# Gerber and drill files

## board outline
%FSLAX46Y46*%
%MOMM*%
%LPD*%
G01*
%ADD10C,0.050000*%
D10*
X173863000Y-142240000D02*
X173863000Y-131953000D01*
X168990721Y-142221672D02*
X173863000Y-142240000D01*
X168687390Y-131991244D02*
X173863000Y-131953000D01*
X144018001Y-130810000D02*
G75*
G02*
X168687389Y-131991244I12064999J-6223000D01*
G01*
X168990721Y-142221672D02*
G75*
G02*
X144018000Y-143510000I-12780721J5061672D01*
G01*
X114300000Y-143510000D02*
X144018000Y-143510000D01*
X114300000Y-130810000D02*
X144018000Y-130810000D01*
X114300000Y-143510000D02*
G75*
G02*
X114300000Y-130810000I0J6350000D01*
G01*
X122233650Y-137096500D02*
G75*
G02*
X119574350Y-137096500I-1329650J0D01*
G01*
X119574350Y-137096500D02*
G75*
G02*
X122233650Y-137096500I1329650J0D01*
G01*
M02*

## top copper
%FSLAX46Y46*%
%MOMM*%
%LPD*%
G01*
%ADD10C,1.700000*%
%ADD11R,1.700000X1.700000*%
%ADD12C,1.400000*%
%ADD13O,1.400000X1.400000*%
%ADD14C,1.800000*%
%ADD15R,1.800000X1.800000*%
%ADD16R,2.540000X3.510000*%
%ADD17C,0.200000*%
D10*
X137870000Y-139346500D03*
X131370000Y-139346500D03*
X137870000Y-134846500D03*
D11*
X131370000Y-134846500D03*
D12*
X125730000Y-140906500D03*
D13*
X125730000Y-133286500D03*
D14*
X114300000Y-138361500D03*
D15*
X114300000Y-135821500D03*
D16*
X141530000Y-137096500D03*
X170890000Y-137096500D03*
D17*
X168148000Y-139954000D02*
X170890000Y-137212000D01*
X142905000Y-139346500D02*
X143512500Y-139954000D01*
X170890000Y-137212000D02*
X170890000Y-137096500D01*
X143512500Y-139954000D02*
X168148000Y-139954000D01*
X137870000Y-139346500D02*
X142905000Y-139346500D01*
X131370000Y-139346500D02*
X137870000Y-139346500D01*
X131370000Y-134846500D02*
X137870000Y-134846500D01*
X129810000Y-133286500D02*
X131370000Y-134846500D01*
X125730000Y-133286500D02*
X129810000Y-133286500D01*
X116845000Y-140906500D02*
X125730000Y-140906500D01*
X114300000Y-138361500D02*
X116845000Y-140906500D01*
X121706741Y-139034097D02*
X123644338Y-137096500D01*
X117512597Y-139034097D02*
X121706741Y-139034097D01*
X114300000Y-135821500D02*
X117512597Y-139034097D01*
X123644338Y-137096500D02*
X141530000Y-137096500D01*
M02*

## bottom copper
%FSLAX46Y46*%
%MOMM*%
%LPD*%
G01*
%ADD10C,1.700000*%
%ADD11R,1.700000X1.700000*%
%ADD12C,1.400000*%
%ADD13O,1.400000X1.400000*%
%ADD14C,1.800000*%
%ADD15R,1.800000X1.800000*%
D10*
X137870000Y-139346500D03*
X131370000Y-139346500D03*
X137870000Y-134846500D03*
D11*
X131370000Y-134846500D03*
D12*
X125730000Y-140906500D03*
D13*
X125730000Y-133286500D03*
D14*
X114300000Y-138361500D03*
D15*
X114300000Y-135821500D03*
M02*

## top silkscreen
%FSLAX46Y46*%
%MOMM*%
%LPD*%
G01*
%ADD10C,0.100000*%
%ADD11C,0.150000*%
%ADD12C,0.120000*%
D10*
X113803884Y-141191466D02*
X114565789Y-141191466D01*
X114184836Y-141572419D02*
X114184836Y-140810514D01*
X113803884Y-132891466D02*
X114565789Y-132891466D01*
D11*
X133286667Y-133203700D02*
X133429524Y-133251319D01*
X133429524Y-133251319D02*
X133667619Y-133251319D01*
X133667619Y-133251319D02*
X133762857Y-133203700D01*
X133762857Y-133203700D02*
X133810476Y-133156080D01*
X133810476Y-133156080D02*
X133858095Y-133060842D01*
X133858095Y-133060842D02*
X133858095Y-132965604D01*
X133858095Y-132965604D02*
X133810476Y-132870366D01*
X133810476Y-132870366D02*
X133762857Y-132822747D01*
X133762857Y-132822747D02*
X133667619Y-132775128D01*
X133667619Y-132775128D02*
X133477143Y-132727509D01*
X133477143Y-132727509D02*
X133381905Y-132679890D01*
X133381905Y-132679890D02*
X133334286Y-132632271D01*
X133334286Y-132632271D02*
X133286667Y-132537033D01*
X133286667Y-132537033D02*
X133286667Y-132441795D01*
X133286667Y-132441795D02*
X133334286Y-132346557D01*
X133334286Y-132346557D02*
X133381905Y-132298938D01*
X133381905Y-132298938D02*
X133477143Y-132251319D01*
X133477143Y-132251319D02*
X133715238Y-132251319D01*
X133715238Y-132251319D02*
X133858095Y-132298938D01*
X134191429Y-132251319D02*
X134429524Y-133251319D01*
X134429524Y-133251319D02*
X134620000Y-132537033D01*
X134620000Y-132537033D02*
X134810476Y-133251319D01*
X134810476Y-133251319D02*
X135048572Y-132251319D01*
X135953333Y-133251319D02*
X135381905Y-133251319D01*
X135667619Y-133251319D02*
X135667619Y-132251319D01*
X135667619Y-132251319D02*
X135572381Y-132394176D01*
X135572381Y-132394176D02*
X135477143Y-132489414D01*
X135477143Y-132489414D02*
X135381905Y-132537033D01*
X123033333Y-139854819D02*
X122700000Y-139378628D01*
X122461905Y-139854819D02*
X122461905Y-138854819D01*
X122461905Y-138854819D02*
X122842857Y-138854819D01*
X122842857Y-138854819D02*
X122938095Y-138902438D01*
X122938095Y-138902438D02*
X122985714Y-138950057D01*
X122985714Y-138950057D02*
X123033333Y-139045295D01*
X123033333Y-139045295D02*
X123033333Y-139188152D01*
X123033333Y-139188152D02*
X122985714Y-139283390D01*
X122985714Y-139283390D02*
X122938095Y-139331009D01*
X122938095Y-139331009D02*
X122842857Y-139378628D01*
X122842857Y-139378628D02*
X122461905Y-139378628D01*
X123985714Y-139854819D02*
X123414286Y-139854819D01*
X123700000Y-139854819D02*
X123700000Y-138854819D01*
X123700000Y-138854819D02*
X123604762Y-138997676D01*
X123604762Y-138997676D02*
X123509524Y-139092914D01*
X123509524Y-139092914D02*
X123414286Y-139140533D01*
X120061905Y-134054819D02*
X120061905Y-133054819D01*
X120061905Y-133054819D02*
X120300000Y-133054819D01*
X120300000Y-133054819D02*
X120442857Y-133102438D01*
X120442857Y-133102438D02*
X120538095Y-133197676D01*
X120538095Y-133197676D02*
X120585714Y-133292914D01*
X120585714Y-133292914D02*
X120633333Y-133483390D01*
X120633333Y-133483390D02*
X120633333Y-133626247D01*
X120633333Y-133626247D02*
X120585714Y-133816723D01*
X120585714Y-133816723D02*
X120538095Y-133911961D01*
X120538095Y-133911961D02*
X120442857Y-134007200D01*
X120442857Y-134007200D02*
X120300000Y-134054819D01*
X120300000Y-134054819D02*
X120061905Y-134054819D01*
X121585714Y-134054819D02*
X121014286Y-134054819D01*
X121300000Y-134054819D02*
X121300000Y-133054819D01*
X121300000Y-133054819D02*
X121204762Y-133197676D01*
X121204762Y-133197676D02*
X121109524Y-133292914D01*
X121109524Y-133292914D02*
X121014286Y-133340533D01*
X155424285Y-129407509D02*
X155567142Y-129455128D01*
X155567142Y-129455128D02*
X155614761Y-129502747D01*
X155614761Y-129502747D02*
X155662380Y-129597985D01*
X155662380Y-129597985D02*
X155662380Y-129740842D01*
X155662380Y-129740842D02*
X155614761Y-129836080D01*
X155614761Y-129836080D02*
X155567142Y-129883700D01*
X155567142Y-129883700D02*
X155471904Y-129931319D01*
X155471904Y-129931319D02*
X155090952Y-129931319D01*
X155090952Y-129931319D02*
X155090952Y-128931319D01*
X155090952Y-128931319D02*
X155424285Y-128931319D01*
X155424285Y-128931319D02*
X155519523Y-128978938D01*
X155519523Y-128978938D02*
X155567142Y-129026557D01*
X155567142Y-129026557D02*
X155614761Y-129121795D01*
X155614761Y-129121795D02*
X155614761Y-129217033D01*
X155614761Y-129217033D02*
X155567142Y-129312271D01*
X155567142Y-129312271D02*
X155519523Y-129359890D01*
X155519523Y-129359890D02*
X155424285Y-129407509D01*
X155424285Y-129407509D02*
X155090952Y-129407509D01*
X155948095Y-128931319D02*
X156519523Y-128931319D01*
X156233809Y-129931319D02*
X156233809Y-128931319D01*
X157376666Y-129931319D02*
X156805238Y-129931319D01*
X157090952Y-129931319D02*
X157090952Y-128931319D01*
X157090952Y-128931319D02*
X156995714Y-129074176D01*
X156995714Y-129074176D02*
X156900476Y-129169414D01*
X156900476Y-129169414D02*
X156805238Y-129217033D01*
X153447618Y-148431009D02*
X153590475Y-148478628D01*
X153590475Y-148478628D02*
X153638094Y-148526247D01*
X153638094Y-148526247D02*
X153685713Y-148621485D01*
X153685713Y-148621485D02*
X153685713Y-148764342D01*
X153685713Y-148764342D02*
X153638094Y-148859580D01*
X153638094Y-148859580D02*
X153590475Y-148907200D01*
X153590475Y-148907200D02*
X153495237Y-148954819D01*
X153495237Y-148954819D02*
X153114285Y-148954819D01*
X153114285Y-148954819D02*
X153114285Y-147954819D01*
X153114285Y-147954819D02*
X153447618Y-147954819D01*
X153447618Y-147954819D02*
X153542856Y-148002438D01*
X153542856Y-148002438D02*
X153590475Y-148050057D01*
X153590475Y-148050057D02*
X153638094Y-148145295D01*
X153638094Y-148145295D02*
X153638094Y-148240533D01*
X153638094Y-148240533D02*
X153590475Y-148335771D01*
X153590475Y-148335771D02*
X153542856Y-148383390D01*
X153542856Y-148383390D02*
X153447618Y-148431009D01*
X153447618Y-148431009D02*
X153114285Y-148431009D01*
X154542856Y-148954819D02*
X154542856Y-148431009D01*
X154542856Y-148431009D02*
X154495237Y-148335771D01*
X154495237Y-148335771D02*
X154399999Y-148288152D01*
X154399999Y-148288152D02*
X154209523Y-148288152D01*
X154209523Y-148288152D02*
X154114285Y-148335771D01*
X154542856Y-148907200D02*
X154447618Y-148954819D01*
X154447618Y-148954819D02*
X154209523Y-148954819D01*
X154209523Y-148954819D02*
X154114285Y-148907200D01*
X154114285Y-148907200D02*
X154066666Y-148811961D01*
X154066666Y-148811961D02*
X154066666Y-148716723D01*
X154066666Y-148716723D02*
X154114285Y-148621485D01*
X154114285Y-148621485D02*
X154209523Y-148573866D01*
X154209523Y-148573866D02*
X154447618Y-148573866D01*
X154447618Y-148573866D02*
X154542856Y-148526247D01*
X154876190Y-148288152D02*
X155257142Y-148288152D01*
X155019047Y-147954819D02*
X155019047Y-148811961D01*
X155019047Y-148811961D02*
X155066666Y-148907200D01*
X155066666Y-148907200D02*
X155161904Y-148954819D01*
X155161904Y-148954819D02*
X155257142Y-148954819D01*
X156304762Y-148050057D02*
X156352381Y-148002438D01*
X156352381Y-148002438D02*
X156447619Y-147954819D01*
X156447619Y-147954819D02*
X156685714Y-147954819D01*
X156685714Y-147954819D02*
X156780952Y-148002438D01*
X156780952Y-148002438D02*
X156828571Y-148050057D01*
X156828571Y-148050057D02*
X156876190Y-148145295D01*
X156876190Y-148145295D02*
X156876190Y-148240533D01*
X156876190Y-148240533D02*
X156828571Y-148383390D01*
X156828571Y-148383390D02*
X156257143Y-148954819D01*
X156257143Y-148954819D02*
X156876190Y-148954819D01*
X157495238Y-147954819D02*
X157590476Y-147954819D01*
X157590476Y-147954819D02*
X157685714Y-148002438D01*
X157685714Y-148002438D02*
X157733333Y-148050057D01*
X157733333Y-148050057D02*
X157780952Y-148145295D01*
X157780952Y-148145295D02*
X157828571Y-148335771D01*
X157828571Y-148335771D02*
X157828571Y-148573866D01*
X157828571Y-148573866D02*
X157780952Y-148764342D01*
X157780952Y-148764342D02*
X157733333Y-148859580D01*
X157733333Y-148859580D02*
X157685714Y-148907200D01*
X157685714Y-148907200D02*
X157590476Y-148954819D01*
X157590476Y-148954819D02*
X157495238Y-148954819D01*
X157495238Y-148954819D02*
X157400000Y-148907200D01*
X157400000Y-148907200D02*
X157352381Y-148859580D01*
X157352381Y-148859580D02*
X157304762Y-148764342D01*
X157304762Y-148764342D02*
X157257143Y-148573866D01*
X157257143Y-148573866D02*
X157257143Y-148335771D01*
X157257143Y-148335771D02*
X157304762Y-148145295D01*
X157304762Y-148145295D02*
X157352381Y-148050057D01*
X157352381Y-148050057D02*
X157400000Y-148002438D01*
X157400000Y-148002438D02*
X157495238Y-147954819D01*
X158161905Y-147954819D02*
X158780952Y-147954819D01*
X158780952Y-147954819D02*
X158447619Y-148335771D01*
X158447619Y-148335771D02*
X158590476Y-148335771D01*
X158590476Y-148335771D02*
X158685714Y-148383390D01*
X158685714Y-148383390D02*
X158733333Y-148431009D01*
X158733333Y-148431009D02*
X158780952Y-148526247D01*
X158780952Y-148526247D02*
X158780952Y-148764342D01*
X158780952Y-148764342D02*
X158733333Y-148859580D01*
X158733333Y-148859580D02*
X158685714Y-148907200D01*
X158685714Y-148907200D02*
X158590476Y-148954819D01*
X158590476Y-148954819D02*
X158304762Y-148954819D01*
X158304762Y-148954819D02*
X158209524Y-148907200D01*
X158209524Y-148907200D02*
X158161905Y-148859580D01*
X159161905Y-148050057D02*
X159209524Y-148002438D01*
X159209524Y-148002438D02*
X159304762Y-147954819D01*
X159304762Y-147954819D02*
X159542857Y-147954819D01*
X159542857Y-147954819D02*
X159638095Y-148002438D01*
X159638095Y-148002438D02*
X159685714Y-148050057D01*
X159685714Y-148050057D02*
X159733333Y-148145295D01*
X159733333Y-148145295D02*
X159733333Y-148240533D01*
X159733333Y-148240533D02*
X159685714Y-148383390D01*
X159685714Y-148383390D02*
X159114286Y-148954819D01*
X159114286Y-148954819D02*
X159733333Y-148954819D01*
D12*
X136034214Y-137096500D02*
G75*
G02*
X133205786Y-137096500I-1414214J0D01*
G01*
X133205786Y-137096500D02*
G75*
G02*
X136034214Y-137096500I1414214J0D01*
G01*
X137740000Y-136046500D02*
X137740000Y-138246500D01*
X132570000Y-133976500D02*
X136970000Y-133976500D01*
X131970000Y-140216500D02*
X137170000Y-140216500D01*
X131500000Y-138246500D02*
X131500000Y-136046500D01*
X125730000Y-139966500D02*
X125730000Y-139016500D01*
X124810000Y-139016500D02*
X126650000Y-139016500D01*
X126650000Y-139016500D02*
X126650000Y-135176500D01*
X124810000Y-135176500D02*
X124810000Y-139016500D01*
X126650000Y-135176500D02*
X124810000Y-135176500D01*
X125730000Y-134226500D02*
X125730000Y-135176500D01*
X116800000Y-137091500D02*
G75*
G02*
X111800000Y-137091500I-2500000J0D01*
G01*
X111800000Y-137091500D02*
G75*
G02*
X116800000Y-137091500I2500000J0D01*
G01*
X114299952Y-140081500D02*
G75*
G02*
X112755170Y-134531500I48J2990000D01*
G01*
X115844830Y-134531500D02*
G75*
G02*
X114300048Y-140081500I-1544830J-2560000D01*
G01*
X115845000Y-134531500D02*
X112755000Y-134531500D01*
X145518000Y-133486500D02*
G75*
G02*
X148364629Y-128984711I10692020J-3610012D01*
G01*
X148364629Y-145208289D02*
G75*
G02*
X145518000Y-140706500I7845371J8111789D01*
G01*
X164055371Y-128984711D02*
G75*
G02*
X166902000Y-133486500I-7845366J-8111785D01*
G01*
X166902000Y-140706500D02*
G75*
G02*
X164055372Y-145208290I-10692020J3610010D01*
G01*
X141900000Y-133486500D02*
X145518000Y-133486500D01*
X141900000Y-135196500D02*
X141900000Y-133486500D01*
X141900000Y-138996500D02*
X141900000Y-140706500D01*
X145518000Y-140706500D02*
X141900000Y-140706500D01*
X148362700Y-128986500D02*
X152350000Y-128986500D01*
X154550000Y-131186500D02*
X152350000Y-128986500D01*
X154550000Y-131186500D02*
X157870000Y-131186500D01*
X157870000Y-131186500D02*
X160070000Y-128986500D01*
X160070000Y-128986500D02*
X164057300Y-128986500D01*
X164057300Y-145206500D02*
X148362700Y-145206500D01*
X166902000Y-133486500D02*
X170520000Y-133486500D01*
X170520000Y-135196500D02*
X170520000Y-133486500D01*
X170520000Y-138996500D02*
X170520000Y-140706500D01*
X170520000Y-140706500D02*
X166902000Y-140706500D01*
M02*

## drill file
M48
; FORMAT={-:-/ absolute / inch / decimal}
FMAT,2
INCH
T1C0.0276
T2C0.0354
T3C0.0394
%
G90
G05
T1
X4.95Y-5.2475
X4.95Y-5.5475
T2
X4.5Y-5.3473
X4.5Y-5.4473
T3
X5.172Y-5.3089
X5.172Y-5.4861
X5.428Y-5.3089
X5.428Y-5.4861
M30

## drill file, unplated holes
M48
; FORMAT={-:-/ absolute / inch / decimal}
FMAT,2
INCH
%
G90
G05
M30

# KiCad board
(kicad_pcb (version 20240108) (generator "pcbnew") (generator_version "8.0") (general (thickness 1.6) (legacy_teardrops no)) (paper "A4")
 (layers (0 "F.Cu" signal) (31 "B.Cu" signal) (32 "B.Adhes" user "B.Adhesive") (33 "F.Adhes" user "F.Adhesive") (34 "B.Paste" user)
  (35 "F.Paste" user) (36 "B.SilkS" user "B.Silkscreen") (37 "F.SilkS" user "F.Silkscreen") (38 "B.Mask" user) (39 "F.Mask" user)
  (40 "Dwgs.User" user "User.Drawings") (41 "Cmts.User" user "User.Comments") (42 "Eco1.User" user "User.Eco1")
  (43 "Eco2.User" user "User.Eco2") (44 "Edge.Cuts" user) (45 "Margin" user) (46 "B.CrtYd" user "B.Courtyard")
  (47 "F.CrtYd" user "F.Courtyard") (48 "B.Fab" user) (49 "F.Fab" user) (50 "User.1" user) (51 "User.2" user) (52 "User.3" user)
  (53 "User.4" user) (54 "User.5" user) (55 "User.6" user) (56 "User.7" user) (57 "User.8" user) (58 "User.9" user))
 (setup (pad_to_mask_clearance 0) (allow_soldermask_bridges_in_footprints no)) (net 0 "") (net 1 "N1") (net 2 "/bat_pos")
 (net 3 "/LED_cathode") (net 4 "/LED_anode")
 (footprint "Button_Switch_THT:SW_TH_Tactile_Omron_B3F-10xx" (layer "F.Cu") (at 131.37 134.8465)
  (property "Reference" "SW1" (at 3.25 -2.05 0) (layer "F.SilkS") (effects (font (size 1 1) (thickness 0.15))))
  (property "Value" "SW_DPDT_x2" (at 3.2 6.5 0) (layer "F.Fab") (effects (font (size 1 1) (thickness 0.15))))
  (fp_line (start 0.13 3.4) (end 0.13 1.2) (stroke (width 0.12) (type solid)) (layer "F.SilkS"))
  (fp_line (start 0.6 5.37) (end 5.8 5.37) (stroke (width 0.12) (type solid)) (layer "F.SilkS"))
  (fp_line (start 1.2 -0.87) (end 5.6 -0.87) (stroke (width 0.12) (type solid)) (layer "F.SilkS"))
  (fp_line (start 6.37 1.2) (end 6.37 3.4) (stroke (width 0.12) (type solid)) (layer "F.SilkS"))
  (fp_circle (center 3.25 2.25) (end 4.25 3.25) (stroke (width 0.12) (type solid)) (fill none) (layer "F.SilkS"))
  (pad "1" thru_hole rect (at 0 0) (size 1.7 1.7) (drill 1) (layers "*.Cu" "*.Mask") (remove_unused_layers no) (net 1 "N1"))
  (pad "1" thru_hole circle (at 6.5 0) (size 1.7 1.7) (drill 1) (layers "*.Cu" "*.Mask") (remove_unused_layers no) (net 1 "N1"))
  (pad "2" thru_hole circle (at 0 4.5) (size 1.7 1.7) (drill 1) (layers "*.Cu" "*.Mask") (remove_unused_layers no) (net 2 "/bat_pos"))
  (pad "2" thru_hole circle (at 6.5 4.5) (size 1.7 1.7) (drill 1) (layers "*.Cu" "*.Mask") (remove_unused_layers no) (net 2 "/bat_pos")))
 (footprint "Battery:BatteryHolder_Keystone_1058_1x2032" (layer "F.Cu") (at 156.21 137.0965 180)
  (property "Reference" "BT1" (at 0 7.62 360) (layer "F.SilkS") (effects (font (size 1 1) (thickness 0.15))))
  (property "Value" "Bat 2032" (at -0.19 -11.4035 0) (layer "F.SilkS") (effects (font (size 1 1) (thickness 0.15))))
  (fp_line (start 14.31 3.61) (end 10.692 3.61) (stroke (width 0.12) (type solid)) (layer "F.SilkS"))
  (fp_line (start 14.31 1.9) (end 14.31 3.61) (stroke (width 0.12) (type solid)) (layer "F.SilkS"))
  (fp_line (start 14.31 -1.9) (end 14.31 -3.61) (stroke (width 0.12) (type solid)) (layer "F.SilkS"))
  (fp_line (start 10.692 -3.61) (end 14.31 -3.61) (stroke (width 0.12) (type solid)) (layer "F.SilkS"))
  (fp_line (start 7.8473 8.11) (end 3.86 8.11) (stroke (width 0.12) (type solid)) (layer "F.SilkS"))
  (fp_line (start 1.66 5.91) (end 3.86 8.11) (stroke (width 0.12) (type solid)) (layer "F.SilkS"))
  (fp_line (start 1.66 5.91) (end -1.66 5.91) (stroke (width 0.12) (type solid)) (layer "F.SilkS"))
  (fp_line (start -1.66 5.91) (end -3.86 8.11) (stroke (width 0.12) (type solid)) (layer "F.SilkS"))
  (fp_line (start -3.86 8.11) (end -7.8473 8.11) (stroke (width 0.12) (type solid)) (layer "F.SilkS"))
  (fp_line (start -7.8473 -8.11) (end 7.8473 -8.11) (stroke (width 0.12) (type solid)) (layer "F.SilkS"))
  (fp_line (start -10.692 3.61) (end -14.31 3.61) (stroke (width 0.12) (type solid)) (layer "F.SilkS"))
  (fp_line (start -14.31 1.9) (end -14.31 3.61) (stroke (width 0.12) (type solid)) (layer "F.SilkS"))
  (fp_line (start -14.31 -1.9) (end -14.31 -3.61) (stroke (width 0.12) (type solid)) (layer "F.SilkS"))
  (fp_line (start -14.31 -3.61) (end -10.692 -3.61) (stroke (width 0.12) (type solid)) (layer "F.SilkS"))
  (fp_arc (start 10.692 3.61) (mid 9.538084 6.031244) (end 7.845371 8.111789) (stroke (width 0.12) (type solid)) (layer "F.SilkS"))
  (fp_arc (start 7.845371 -8.111789) (mid 9.538085 -6.031244) (end 10.692 -3.61) (stroke (width 0.12) (type solid)) (layer "F.SilkS"))
  (fp_arc (start -7.845371 8.111789) (mid -9.538085 6.031244) (end -10.692 3.61) (stroke (width 0.12) (type solid)) (layer "F.SilkS"))
  (fp_arc (start -10.692 -3.61) (mid -9.538084 -6.031244) (end -7.845371 -8.111789) (stroke (width 0.12) (type solid)) (layer "F.SilkS"))
  (pad "1" smd rect (at -14.68 0 180) (size 2.54 3.51) (layers "F.Cu" "F.Paste" "F.Mask") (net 2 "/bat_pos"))
  (pad "2" smd rect (at 14.68 0 180) (size 2.54 3.51) (layers "F.Cu" "F.Paste" "F.Mask") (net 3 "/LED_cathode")))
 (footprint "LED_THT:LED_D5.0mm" (layer "F.Cu") (at 114.3 135.8215 -90)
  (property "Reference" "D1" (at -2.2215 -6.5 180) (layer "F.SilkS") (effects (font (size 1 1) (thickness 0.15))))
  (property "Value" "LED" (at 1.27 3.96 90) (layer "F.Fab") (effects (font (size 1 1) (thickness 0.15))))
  (fp_line (start -1.29 -1.545) (end -1.29 1.545) (stroke (width 0.12) (type solid)) (layer "F.SilkS"))
  (fp_arc (start 4.26 0.000048) (mid 2.071756 2.880501) (end -1.29 1.54483) (stroke (width 0.12) (type solid)) (layer "F.SilkS"))
  (fp_arc (start -1.29 -1.54483) (mid 2.071756 -2.880501) (end 4.26 -0.000048) (stroke (width 0.12) (type solid)) (layer "F.SilkS"))
  (fp_circle (center 1.27 0) (end 3.77 0) (stroke (width 0.12) (type solid)) (fill none) (layer "F.SilkS"))
  (pad "1" thru_hole rect (at 0 0 270) (size 1.8 1.8) (drill 0.9) (layers "*.Cu" "*.Mask") (remove_unused_layers no) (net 3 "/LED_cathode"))
  (pad "2" thru_hole circle (at 2.54 0 270) (size 1.8 1.8) (drill 0.9) (layers "*.Cu" "*.Mask") (remove_unused_layers no)
   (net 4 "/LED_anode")))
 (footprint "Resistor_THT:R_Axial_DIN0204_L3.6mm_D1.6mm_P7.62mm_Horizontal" (layer "F.Cu") (at 125.73 140.9065 90)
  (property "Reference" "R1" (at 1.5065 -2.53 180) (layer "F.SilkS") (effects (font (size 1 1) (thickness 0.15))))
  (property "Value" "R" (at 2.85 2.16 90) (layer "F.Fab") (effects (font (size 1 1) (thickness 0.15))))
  (fp_line (start 5.73 -0.92) (end 1.89 -0.92) (stroke (width 0.12) (type solid)) (layer "F.SilkS"))
  (fp_line (start 1.89 -0.92) (end 1.89 0.92) (stroke (width 0.12) (type solid)) (layer "F.SilkS"))
  (fp_line (start 6.68 0) (end 5.73 0) (stroke (width 0.12) (type solid)) (layer "F.SilkS"))
  (fp_line (start 0.94 0) (end 1.89 0) (stroke (width 0.12) (type solid)) (layer "F.SilkS"))
  (fp_line (start 5.73 0.92) (end 5.73 -0.92) (stroke (width 0.12) (type solid)) (layer "F.SilkS"))
  (fp_line (start 1.89 0.92) (end 5.73 0.92) (stroke (width 0.12) (type solid)) (layer "F.SilkS"))
  (pad "1" thru_hole circle (at 0 0 90) (size 1.4 1.4) (drill 0.7) (layers "*.Cu" "*.Mask") (remove_unused_layers no) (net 4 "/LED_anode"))
  (pad "2" thru_hole oval (at 7.62 0 90) (size 1.4 1.4) (drill 0.7) (layers "*.Cu" "*.Mask") (remove_unused_layers no) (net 1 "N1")))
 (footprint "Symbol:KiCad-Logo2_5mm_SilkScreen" (layer "B.Cu") (at 156.21 132.76 180)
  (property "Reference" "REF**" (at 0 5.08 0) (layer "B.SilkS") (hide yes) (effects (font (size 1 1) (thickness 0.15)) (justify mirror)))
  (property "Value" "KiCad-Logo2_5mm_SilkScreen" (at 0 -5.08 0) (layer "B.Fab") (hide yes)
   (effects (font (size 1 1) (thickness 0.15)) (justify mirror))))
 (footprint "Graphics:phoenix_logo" (layer "B.Cu") (at 156.45 141.24 180)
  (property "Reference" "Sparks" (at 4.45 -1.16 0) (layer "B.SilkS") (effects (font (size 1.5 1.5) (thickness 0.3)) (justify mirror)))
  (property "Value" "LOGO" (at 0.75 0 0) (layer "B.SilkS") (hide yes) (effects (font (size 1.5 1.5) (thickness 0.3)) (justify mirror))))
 (gr_line (start 114.3 143.51) (end 144.018 143.51) (locked yes) (stroke (width 0.05) (type default)) (layer "Edge.Cuts"))
 (gr_line (start 114.3 130.81) (end 144.018 130.81) (locked yes) (stroke (width 0.05) (type default)) (layer "Edge.Cuts"))
 (gr_line (start 168.68739 131.991244) (end 173.863 131.953) (locked yes) (stroke (width 0.05) (type default)) (layer "Edge.Cuts"))
 (gr_line (start 168.990721 142.221672) (end 173.863 142.24) (locked yes) (stroke (width 0.05) (type default)) (layer "Edge.Cuts"))
 (gr_arc (start 168.990721 142.221672) (mid 156.918234 150.888283) (end 144.018 143.51) (locked yes) (stroke (width 0.05) (type default))
  (layer "Edge.Cuts"))
 (gr_circle (center 120.904 137.0965) (end 120.396 135.867718) (stroke (width 0.05) (type default)) (fill none) (layer "Edge.Cuts"))
 (gr_line (start 173.863 142.24) (end 173.863 131.953) (locked yes) (stroke (width 0.05) (type default)) (layer "Edge.Cuts"))
 (gr_arc (start 144.018001 130.81) (mid 156.732284 123.473193) (end 168.68739 131.991244) (locked yes) (stroke (width 0.05) (type default))
  (layer "Edge.Cuts"))
 (gr_arc (start 114.3 143.51) (mid 107.95 137.16) (end 114.3 130.81) (locked yes) (stroke (width 0.05) (type default)) (layer "Edge.Cuts"))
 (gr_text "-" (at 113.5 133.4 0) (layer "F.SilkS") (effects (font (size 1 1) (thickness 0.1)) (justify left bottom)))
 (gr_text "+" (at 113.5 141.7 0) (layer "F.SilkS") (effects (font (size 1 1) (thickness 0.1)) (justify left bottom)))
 (segment (start 142.905 139.3465) (end 143.5125 139.954) (width 0.2) (layer "F.Cu") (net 2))
 (segment (start 137.87 139.3465) (end 142.905 139.3465) (width 0.2) (layer "F.Cu") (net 2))
 (segment (start 143.5125 139.954) (end 168.148 139.954) (width 0.2) (layer "F.Cu") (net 2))
 (segment (start 131.37 139.3465) (end 137.87 139.3465) (width 0.2) (layer "F.Cu") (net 2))
 (segment (start 170.89 137.212) (end 170.89 137.0965) (width 0.2) (layer "F.Cu") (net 2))
 (segment (start 168.148 139.954) (end 170.89 137.212) (width 0.2) (layer "F.Cu") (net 2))
 (segment (start 123.644338 137.0965) (end 141.53 137.0965) (width 0.2) (layer "F.Cu") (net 3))
 (segment (start 114.3 135.8215) (end 117.512597 139.034097) (width 0.2) (layer "F.Cu") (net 3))
 (segment (start 117.512597 139.034097) (end 121.706741 139.034097) (width 0.2) (layer "F.Cu") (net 3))
 (segment (start 121.706741 139.034097) (end 123.644338 137.0965) (width 0.2) (layer "F.Cu") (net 3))
 (segment (start 116.845 140.9065) (end 125.73 140.9065) (width 0.2) (layer "F.Cu") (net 4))
 (segment (start 114.3 138.3615) (end 116.845 140.9065) (width 0.2) (layer "F.Cu") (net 4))
 (segment (start 131.37 134.8465) (end 137.87 134.8465) (width 0.2) (layer "F.Cu") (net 1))
 (segment (start 129.81 133.2865) (end 131.37 134.8465) (width 0.2) (layer "F.Cu") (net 1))
 (segment (start 125.73 133.2865) (end 129.81 133.2865) (width 0.2) (layer "F.Cu") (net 1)))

